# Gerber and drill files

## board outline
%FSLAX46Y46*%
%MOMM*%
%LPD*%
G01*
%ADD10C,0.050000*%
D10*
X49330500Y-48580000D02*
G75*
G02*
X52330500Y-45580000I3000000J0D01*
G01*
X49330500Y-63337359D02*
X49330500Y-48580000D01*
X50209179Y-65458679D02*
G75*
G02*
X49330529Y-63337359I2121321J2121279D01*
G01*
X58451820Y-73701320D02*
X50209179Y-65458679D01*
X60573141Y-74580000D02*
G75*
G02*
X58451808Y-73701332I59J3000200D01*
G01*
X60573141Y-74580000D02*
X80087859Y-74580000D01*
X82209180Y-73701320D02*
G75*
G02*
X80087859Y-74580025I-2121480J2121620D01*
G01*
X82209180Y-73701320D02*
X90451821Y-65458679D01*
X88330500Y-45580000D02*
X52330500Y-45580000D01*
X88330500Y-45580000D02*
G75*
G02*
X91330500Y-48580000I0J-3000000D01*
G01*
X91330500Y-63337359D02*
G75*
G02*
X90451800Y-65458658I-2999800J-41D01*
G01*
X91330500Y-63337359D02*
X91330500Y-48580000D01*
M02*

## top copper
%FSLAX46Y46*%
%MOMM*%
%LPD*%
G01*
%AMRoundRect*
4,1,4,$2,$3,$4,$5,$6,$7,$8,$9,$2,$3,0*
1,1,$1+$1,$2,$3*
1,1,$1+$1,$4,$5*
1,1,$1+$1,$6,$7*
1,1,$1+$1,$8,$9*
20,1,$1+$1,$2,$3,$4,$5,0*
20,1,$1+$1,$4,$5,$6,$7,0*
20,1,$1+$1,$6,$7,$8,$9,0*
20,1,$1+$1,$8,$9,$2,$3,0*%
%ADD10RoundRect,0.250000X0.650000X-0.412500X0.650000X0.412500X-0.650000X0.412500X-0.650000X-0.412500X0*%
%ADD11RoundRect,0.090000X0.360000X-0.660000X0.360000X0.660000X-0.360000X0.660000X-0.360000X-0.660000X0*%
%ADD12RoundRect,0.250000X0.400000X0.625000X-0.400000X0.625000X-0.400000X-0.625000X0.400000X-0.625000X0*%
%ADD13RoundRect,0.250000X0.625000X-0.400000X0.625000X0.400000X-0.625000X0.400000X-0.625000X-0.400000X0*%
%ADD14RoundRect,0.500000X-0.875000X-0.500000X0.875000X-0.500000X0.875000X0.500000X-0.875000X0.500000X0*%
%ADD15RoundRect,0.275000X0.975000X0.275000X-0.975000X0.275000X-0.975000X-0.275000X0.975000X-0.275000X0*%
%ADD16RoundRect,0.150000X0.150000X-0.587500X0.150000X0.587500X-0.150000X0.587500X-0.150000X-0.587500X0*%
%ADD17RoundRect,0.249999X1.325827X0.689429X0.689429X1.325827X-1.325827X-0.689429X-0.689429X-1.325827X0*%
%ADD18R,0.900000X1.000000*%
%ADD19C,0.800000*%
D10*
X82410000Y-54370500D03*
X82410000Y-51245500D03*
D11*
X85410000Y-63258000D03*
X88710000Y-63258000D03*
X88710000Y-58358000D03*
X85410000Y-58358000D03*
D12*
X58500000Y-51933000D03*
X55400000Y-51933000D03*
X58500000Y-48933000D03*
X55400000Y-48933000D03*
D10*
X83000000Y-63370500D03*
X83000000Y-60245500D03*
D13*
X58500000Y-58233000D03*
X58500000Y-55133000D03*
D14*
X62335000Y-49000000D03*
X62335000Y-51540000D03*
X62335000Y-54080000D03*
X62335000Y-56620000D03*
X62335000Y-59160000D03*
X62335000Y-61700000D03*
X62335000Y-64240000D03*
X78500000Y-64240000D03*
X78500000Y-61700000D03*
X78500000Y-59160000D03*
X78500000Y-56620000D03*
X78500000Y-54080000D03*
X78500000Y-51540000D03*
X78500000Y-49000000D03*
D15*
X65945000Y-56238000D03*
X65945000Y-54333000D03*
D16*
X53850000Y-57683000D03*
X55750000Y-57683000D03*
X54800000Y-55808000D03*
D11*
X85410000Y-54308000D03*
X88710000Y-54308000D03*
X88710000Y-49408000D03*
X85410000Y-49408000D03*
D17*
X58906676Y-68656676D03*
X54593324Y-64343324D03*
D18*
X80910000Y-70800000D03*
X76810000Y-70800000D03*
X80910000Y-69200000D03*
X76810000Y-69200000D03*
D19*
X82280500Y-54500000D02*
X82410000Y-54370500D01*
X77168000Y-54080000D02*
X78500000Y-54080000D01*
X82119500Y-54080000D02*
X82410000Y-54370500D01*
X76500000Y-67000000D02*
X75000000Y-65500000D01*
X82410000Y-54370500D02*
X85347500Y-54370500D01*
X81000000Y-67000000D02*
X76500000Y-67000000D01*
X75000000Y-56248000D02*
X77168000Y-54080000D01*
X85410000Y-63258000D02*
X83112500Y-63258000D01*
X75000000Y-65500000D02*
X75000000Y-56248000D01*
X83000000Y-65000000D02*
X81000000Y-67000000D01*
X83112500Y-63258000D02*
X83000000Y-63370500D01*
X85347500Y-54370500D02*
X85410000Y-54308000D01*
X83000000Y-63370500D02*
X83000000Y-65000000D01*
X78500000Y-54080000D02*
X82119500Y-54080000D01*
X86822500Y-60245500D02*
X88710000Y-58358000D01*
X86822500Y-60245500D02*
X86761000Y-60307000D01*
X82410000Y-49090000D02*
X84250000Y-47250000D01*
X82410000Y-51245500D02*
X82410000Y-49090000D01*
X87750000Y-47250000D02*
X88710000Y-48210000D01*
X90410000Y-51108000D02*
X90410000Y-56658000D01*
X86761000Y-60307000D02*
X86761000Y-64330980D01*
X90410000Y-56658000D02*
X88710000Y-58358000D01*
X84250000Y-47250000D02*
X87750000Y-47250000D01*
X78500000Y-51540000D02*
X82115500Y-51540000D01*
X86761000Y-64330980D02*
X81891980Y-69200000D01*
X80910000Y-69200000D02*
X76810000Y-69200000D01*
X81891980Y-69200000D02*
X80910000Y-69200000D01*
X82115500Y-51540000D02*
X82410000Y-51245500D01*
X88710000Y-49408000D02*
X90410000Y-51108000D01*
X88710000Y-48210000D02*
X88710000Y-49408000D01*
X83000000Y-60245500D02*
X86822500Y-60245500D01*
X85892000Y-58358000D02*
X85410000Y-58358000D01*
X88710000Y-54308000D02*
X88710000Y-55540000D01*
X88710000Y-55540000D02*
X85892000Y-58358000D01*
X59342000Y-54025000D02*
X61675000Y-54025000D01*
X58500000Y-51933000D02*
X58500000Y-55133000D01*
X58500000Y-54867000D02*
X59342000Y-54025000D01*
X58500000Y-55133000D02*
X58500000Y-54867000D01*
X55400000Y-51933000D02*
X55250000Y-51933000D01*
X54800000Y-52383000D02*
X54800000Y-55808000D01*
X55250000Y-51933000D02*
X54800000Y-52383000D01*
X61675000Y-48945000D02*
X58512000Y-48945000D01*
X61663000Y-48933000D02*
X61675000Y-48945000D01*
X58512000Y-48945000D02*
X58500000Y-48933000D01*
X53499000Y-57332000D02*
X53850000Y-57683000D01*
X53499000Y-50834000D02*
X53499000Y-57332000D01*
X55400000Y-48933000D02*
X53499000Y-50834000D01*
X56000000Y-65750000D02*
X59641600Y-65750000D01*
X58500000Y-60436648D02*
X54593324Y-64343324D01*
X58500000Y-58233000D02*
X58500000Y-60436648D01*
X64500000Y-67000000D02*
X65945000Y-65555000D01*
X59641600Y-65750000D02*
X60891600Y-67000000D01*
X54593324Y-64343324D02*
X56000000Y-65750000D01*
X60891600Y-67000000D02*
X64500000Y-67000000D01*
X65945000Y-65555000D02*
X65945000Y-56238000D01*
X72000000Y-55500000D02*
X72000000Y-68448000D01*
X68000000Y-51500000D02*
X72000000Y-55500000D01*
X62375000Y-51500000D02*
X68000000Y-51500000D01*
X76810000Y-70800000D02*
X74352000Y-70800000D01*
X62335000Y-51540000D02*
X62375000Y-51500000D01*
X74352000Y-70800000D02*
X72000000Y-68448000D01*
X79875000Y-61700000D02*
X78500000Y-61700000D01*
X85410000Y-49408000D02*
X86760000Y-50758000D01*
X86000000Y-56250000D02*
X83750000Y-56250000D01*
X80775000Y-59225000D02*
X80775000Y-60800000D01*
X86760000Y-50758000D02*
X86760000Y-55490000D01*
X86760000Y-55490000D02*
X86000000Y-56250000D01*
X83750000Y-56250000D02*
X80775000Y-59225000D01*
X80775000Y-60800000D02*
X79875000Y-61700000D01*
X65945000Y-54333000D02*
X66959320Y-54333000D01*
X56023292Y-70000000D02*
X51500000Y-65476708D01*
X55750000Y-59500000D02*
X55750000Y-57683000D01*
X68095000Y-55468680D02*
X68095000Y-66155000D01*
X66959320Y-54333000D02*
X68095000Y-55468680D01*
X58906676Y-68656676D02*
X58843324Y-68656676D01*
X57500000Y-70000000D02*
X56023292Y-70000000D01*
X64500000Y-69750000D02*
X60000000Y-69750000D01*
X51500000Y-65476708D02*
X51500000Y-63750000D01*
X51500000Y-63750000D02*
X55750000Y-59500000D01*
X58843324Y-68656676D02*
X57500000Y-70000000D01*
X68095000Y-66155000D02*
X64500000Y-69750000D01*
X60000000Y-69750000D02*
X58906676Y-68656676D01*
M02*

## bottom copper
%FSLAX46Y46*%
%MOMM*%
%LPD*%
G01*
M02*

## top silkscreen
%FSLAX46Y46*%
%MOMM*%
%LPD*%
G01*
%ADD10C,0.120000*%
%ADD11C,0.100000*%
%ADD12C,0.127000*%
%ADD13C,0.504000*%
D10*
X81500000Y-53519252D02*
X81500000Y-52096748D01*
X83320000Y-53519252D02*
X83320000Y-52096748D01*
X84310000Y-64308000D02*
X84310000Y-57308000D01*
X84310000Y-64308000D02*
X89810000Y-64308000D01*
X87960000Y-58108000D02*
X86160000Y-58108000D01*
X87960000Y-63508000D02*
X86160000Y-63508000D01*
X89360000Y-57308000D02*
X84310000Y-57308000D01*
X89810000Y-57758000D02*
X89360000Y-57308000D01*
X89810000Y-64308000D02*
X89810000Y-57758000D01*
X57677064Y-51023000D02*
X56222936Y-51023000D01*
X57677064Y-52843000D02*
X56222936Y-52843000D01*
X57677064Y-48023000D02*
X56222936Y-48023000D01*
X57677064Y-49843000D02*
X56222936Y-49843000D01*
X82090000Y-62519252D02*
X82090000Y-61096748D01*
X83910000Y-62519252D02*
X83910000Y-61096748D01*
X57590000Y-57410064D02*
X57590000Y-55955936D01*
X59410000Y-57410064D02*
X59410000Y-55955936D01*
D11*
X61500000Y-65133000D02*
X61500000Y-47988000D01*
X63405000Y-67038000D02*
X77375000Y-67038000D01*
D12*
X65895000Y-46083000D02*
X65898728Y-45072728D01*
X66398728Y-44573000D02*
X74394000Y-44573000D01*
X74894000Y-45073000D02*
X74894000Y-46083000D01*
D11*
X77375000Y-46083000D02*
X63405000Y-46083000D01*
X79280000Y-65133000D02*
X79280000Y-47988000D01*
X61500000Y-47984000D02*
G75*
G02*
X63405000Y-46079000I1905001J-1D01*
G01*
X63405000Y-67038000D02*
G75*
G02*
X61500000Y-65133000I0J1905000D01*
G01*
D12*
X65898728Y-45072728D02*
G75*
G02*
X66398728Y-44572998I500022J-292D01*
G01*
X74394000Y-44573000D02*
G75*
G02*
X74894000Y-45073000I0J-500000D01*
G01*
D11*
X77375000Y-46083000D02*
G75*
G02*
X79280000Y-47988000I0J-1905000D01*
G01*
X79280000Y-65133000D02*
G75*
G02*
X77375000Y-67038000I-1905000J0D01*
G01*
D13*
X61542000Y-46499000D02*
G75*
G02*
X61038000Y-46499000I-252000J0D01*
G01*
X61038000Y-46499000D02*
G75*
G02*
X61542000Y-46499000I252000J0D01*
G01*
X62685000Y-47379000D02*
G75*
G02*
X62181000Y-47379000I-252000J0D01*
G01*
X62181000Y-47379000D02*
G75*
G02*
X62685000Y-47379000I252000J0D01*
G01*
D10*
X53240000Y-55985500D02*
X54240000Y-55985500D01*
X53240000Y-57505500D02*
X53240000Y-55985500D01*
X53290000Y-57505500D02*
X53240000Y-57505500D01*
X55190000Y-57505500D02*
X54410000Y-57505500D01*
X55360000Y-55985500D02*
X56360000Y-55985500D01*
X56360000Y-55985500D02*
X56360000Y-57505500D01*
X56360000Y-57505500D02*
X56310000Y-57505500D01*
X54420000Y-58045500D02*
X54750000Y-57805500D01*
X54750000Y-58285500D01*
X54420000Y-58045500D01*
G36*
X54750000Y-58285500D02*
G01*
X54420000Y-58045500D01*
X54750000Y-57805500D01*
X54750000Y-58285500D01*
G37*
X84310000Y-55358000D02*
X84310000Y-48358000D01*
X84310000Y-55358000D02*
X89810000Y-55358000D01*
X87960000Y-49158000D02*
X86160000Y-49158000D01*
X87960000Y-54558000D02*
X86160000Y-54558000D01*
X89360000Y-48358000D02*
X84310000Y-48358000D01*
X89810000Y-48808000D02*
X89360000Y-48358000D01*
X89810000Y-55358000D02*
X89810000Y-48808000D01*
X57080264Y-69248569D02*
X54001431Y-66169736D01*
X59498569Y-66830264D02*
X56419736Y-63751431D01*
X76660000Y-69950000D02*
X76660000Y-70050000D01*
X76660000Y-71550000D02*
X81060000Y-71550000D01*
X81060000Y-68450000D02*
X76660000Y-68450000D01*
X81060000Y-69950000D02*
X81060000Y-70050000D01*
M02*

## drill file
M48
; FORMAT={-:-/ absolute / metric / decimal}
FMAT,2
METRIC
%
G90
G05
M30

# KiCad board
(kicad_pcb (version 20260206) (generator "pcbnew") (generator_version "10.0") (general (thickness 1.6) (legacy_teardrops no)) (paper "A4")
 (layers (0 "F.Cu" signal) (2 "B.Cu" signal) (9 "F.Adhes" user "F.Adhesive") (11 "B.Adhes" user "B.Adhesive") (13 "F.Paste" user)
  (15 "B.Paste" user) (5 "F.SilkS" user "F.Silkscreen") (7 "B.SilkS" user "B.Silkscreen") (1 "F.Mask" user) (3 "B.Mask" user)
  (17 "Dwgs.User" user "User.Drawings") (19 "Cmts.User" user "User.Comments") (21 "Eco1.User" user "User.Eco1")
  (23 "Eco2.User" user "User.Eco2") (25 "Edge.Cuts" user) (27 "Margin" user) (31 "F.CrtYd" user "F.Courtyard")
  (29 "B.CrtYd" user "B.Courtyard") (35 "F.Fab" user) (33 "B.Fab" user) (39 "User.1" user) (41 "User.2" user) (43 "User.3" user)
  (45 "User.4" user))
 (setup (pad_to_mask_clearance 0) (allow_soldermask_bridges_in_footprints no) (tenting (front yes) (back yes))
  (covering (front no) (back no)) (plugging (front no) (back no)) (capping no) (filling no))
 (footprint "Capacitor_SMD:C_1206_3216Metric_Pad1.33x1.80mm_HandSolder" (layer "F.Cu") (at 82.41 52.808 90)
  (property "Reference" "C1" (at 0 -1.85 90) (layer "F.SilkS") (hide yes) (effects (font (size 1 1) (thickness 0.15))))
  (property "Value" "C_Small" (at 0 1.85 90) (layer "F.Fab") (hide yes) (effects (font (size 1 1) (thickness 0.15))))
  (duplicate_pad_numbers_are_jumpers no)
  (fp_line (start -0.711252 -0.91) (end 0.711252 -0.91) (stroke (width 0.12) (type solid)) (layer "F.SilkS"))
  (fp_line (start -0.711252 0.91) (end 0.711252 0.91) (stroke (width 0.12) (type solid)) (layer "F.SilkS"))
  (pad "1" smd roundrect (at -1.5625 0 90) (size 1.325 1.8) (layers "F.Cu" "F.Mask" "F.Paste") (roundrect_rratio 0.188679) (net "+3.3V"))
  (pad "2" smd roundrect (at 1.5625 0 90) (size 1.325 1.8) (layers "F.Cu" "F.Mask" "F.Paste") (roundrect_rratio 0.188679) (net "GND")))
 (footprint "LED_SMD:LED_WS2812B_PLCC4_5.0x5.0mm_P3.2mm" (layer "F.Cu") (at 87.06 60.808 90)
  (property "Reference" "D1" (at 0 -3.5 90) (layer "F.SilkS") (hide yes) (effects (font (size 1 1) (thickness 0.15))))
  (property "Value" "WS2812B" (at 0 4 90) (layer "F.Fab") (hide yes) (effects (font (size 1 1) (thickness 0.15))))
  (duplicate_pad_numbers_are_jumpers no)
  (fp_line (start -3.5 -2.75) (end 3.5 -2.75) (stroke (width 0.12) (type solid)) (layer "F.SilkS"))
  (fp_line (start -3.5 -2.75) (end -3.5 2.75) (stroke (width 0.12) (type default)) (layer "F.SilkS"))
  (fp_line (start 2.7 0.9) (end 2.7 -0.9) (stroke (width 0.12) (type default)) (layer "F.SilkS"))
  (fp_line (start -2.7 0.9) (end -2.7 -0.9) (stroke (width 0.12) (type default)) (layer "F.SilkS"))
  (fp_line (start 3.5 2.3) (end 3.5 -2.75) (stroke (width 0.12) (type default)) (layer "F.SilkS"))
  (fp_line (start 3.05 2.75) (end 3.5 2.3) (stroke (width 0.12) (type default)) (layer "F.SilkS"))
  (fp_line (start -3.5 2.75) (end 3.05 2.75) (stroke (width 0.12) (type solid)) (layer "F.SilkS"))
  (pad "1" smd roundrect (at -2.45 -1.65 90) (size 1.5 0.9) (layers "F.Cu" "F.Mask" "F.Paste") (roundrect_rratio 0.1) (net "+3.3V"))
  (pad "2" smd roundrect (at -2.45 1.65 90) (size 1.5 0.9) (layers "F.Cu" "F.Mask" "F.Paste") (roundrect_rratio 0.1)
   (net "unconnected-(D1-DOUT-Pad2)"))
  (pad "3" smd roundrect (at 2.45 1.65 90) (size 1.5 0.9) (layers "F.Cu" "F.Mask" "F.Paste") (roundrect_rratio 0.1) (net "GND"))
  (pad "4" smd roundrect (at 2.45 -1.65 90) (size 1.5 0.9) (layers "F.Cu" "F.Mask" "F.Paste") (roundrect_rratio 0.1) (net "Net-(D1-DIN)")))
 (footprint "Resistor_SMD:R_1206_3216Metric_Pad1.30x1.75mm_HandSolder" (layer "F.Cu") (at 56.95 51.933 180)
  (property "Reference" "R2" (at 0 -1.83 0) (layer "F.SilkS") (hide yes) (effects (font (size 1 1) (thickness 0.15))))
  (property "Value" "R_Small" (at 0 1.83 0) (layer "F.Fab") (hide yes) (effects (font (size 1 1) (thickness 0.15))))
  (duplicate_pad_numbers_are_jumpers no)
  (fp_line (start -0.727064 0.91) (end 0.727064 0.91) (stroke (width 0.12) (type solid)) (layer "F.SilkS"))
  (fp_line (start -0.727064 -0.91) (end 0.727064 -0.91) (stroke (width 0.12) (type solid)) (layer "F.SilkS"))
  (pad "1" smd roundrect (at -1.55 0 180) (size 1.3 1.75) (layers "F.Cu" "F.Mask" "F.Paste") (roundrect_rratio 0.192308) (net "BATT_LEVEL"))
  (pad "2" smd roundrect (at 1.55 0 180) (size 1.3 1.75) (layers "F.Cu" "F.Mask" "F.Paste") (roundrect_rratio 0.192308) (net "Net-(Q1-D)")))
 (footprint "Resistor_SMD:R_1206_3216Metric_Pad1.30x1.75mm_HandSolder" (layer "F.Cu") (at 56.95 48.933 180)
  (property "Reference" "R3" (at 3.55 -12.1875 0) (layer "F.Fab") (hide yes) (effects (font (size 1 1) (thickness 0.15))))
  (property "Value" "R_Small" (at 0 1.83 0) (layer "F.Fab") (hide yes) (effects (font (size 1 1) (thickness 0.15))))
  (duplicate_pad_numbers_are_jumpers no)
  (fp_line (start -0.727064 0.91) (end 0.727064 0.91) (stroke (width 0.12) (type solid)) (layer "F.SilkS"))
  (fp_line (start -0.727064 -0.91) (end 0.727064 -0.91) (stroke (width 0.12) (type solid)) (layer "F.SilkS"))
  (pad "1" smd roundrect (at -1.55 0 180) (size 1.3 1.75) (layers "F.Cu" "F.Mask" "F.Paste") (roundrect_rratio 0.192308) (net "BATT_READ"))
  (pad "2" smd roundrect (at 1.55 0 180) (size 1.3 1.75) (layers "F.Cu" "F.Mask" "F.Paste") (roundrect_rratio 0.192308) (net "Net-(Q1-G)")))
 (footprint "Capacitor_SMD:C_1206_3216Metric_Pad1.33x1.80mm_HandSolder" (layer "F.Cu") (at 83 61.808 90)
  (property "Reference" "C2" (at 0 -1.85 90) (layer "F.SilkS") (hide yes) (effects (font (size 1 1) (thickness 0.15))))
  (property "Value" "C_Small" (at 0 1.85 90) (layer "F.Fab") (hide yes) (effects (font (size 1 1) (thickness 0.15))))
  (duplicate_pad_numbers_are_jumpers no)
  (fp_line (start -0.711252 -0.91) (end 0.711252 -0.91) (stroke (width 0.12) (type solid)) (layer "F.SilkS"))
  (fp_line (start -0.711252 0.91) (end 0.711252 0.91) (stroke (width 0.12) (type solid)) (layer "F.SilkS"))
  (pad "1" smd roundrect (at -1.5625 0 90) (size 1.325 1.8) (layers "F.Cu" "F.Mask" "F.Paste") (roundrect_rratio 0.188679) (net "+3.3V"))
  (pad "2" smd roundrect (at 1.5625 0 90) (size 1.325 1.8) (layers "F.Cu" "F.Mask" "F.Paste") (roundrect_rratio 0.188679) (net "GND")))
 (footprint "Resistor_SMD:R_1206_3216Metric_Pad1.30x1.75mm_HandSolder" (layer "F.Cu") (at 58.5 56.683 90)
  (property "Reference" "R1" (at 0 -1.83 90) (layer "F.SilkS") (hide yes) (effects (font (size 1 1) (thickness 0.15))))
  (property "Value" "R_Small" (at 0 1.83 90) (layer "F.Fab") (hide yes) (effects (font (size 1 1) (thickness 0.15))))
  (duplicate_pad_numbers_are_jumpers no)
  (fp_line (start -0.727064 -0.91) (end 0.727064 -0.91) (stroke (width 0.12) (type solid)) (layer "F.SilkS"))
  (fp_line (start -0.727064 0.91) (end 0.727064 0.91) (stroke (width 0.12) (type solid)) (layer "F.SilkS"))
  (pad "1" smd roundrect (at -1.55 0 90) (size 1.3 1.75) (layers "F.Cu" "F.Mask" "F.Paste") (roundrect_rratio 0.192308) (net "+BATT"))
  (pad "2" smd roundrect (at 1.55 0 90) (size 1.3 1.75) (layers "F.Cu" "F.Mask" "F.Paste") (roundrect_rratio 0.192308) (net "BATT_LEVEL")))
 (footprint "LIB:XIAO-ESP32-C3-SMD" (layer "F.Cu") (at 61.5 67.12)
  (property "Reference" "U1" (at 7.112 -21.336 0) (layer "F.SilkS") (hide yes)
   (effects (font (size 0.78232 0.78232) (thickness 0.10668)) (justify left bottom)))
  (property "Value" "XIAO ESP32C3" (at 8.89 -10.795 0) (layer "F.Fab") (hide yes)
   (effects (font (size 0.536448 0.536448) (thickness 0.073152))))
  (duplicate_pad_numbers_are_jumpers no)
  (fp_line (start 0 -1.987) (end 0 -19.132) (stroke (width 0.1) (type solid)) (layer "F.SilkS"))
  (fp_line (start 1.905 -0.082) (end 15.875 -0.082) (stroke (width 0.1) (type solid)) (layer "F.SilkS"))
  (fp_line (start 4.395 -21.037) (end 4.398728 -22.047272) (stroke (width 0.127) (type solid)) (layer "F.SilkS"))
  (fp_line (start 4.898728 -22.547) (end 12.894 -22.547) (stroke (width 0.127) (type solid)) (layer "F.SilkS"))
  (fp_line (start 13.394 -22.047) (end 13.394 -21.037) (stroke (width 0.127) (type solid)) (layer "F.SilkS"))
  (fp_line (start 15.875 -21.037) (end 1.905 -21.037) (stroke (width 0.1) (type solid)) (layer "F.SilkS"))
  (fp_line (start 17.78 -1.987) (end 17.78 -19.132) (stroke (width 0.1) (type solid)) (layer "F.SilkS"))
  (fp_arc (start 0 -19.136) (mid 0.557962 -20.483038) (end 1.905 -21.041) (stroke (width 0.1) (type solid)) (layer "F.SilkS"))
  (fp_arc (start 1.905 -0.082) (mid 0.557962 -0.639962) (end 0 -1.987) (stroke (width 0.1) (type solid)) (layer "F.SilkS"))
  (fp_arc (start 4.398728 -22.047272) (mid 4.545272 -22.40064) (end 4.898728 -22.547) (stroke (width 0.127) (type default))
   (layer "F.SilkS"))
  (fp_arc (start 12.894 -22.547) (mid 13.247553 -22.400553) (end 13.394 -22.047) (stroke (width 0.127) (type default)) (layer "F.SilkS"))
  (fp_arc (start 15.875 -21.037) (mid 17.222038 -20.479038) (end 17.78 -19.132) (stroke (width 0.1) (type solid)) (layer "F.SilkS"))
  (fp_arc (start 17.78 -1.987) (mid 17.222038 -0.639962) (end 15.875 -0.082) (stroke (width 0.1) (type solid)) (layer "F.SilkS"))
  (fp_circle (center -0.21 -20.621) (end -0.21 -20.875) (stroke (width 0.5) (type solid)) (fill yes) (layer "F.SilkS"))
  (fp_circle (center 0.933 -19.741) (end 0.933 -19.995) (stroke (width 0.5) (type solid)) (fill yes) (layer "F.SilkS"))
  (pad "1" smd roundrect (at 0.835 -18.12) (size 2.75 2) (layers "F.Cu" "F.Mask" "F.Paste") (roundrect_rratio 0.25) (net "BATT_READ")
   (solder_mask_margin 0.0508) (thermal_bridge_angle 45))
  (pad "2" smd roundrect (at 0.835 -15.58) (size 2.75 2) (layers "F.Cu" "F.Mask" "F.Paste") (roundrect_rratio 0.25) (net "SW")
   (solder_mask_margin 0.0508) (thermal_bridge_angle 45))
  (pad "3" smd roundrect (at 0.835 -13.04) (size 2.75 2) (layers "F.Cu" "F.Mask" "F.Paste") (roundrect_rratio 0.25) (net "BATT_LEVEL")
   (solder_mask_margin 0.0508) (thermal_bridge_angle 45))
  (pad "4" smd roundrect (at 0.835 -10.5) (size 2.75 2) (layers "F.Cu" "F.Mask" "F.Paste") (roundrect_rratio 0.25)
   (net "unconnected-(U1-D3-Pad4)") (solder_mask_margin 0.0508) (thermal_bridge_angle 45))
  (pad "5" smd roundrect (at 0.835 -7.96) (size 2.75 2) (layers "F.Cu" "F.Mask" "F.Paste") (roundrect_rratio 0.25)
   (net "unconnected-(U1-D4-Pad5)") (solder_mask_margin 0.0508) (thermal_bridge_angle 45))
  (pad "6" smd roundrect (at 0.835 -5.42) (size 2.75 2) (layers "F.Cu" "F.Mask" "F.Paste") (roundrect_rratio 0.25)
   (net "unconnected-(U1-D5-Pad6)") (solder_mask_margin 0.0508) (thermal_bridge_angle 45))
  (pad "7" smd roundrect (at 0.835 -2.88) (size 2.75 2) (layers "F.Cu" "F.Mask" "F.Paste") (roundrect_rratio 0.25)
   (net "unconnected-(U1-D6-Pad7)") (solder_mask_margin 0.0508) (thermal_bridge_angle 45))
  (pad "8" smd roundrect (at 17 -2.88) (size 2.75 2) (layers "F.Cu" "F.Mask" "F.Paste") (roundrect_rratio 0.25)
   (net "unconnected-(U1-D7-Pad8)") (solder_mask_margin 0.0508) (thermal_bridge_angle 45))
  (pad "9" smd roundrect (at 17 -5.42) (size 2.75 2) (layers "F.Cu" "F.Mask" "F.Paste") (roundrect_rratio 0.25) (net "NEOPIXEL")
   (solder_mask_margin 0.0508) (thermal_bridge_angle 45))
  (pad "10" smd roundrect (at 17 -7.96) (size 2.75 2) (layers "F.Cu" "F.Mask" "F.Paste") (roundrect_rratio 0.25)
   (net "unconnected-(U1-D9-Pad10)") (solder_mask_margin 0.0508) (thermal_bridge_angle 45))
  (pad "11" smd roundrect (at 17 -10.5) (size 2.75 2) (layers "F.Cu" "F.Mask" "F.Paste") (roundrect_rratio 0.25)
   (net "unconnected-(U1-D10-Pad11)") (solder_mask_margin 0.0508) (thermal_bridge_angle 45))
  (pad "12" smd roundrect (at 17 -13.04) (size 2.75 2) (layers "F.Cu" "F.Mask" "F.Paste") (roundrect_rratio 0.25) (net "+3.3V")
   (solder_mask_margin 0.0508) (thermal_bridge_angle 45))
  (pad "13" smd roundrect (at 17 -15.58) (size 2.75 2) (layers "F.Cu" "F.Mask" "F.Paste") (roundrect_rratio 0.25) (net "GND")
   (solder_mask_margin 0.0508) (thermal_bridge_angle 45))
  (pad "14" smd roundrect (at 17 -18.12) (size 2.75 2) (layers "F.Cu" "F.Mask" "F.Paste") (roundrect_rratio 0.25)
   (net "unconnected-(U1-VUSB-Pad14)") (solder_mask_margin 0.0508) (thermal_bridge_angle 45))
  (pad "15" smd roundrect (at 4.445 -10.882 180) (size 2.5 1.1) (layers "F.Cu" "F.Mask" "F.Paste") (roundrect_rratio 0.25) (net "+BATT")
   (solder_mask_margin 0.0508) (thermal_bridge_angle 45))
  (pad "16" smd roundrect (at 4.445 -12.787 180) (size 2.5 1.1) (layers "F.Cu" "F.Mask" "F.Paste") (roundrect_rratio 0.25) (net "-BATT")
   (solder_mask_margin 0.0508) (thermal_bridge_angle 45)))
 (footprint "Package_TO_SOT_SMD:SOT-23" (layer "F.Cu") (at 54.8 56.7455 90)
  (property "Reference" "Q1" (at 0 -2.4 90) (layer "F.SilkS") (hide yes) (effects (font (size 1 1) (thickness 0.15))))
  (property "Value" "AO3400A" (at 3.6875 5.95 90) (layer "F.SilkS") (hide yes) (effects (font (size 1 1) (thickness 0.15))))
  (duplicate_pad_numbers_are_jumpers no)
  (fp_line (start 0.76 -1.56) (end 0.76 -0.56) (stroke (width 0.12) (type solid)) (layer "F.SilkS"))
  (fp_line (start -0.76 -1.56) (end 0.76 -1.56) (stroke (width 0.12) (type solid)) (layer "F.SilkS"))
  (fp_line (start -0.76 -1.51) (end -0.76 -1.56) (stroke (width 0.12) (type solid)) (layer "F.SilkS"))
  (fp_line (start -0.76 0.39) (end -0.76 -0.39) (stroke (width 0.12) (type solid)) (layer "F.SilkS"))
  (fp_line (start 0.76 0.56) (end 0.76 1.56) (stroke (width 0.12) (type solid)) (layer "F.SilkS"))
  (fp_line (start 0.76 1.56) (end -0.76 1.56) (stroke (width 0.12) (type solid)) (layer "F.SilkS"))
  (fp_line (start -0.76 1.56) (end -0.76 1.51) (stroke (width 0.12) (type solid)) (layer "F.SilkS"))
  (fp_poly (pts (xy -1.3 -0.38) (xy -1.06 -0.05) (xy -1.54 -0.05)) (stroke (width 0.12) (type solid)) (fill yes) (layer "F.SilkS"))
  (pad "1" smd roundrect (at -0.9375 -0.95 90) (size 1.475 0.6) (layers "F.Cu" "F.Mask" "F.Paste") (roundrect_rratio 0.25)
   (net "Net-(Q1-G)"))
  (pad "2" smd roundrect (at -0.9375 0.95 90) (size 1.475 0.6) (layers "F.Cu" "F.Mask" "F.Paste") (roundrect_rratio 0.25) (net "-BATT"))
  (pad "3" smd roundrect (at 0.9375 0 90) (size 1.475 0.6) (layers "F.Cu" "F.Mask" "F.Paste") (roundrect_rratio 0.25) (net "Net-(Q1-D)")))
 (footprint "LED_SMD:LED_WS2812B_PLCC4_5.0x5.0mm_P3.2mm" (layer "F.Cu") (at 87.06 51.858 90)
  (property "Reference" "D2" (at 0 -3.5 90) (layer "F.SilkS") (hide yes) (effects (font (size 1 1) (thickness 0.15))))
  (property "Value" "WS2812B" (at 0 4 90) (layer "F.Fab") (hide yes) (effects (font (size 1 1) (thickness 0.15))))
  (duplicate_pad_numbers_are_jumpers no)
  (fp_line (start -3.5 -2.75) (end 3.5 -2.75) (stroke (width 0.12) (type solid)) (layer "F.SilkS"))
  (fp_line (start -3.5 -2.75) (end -3.5 2.75) (stroke (width 0.12) (type default)) (layer "F.SilkS"))
  (fp_line (start 2.7 0.9) (end 2.7 -0.9) (stroke (width 0.12) (type default)) (layer "F.SilkS"))
  (fp_line (start -2.7 0.9) (end -2.7 -0.9) (stroke (width 0.12) (type default)) (layer "F.SilkS"))
  (fp_line (start 3.5 2.3) (end 3.5 -2.75) (stroke (width 0.12) (type default)) (layer "F.SilkS"))
  (fp_line (start 3.05 2.75) (end 3.5 2.3) (stroke (width 0.12) (type default)) (layer "F.SilkS"))
  (fp_line (start -3.5 2.75) (end 3.05 2.75) (stroke (width 0.12) (type solid)) (layer "F.SilkS"))
  (pad "1" smd roundrect (at -2.45 -1.65 90) (size 1.5 0.9) (layers "F.Cu" "F.Mask" "F.Paste") (roundrect_rratio 0.1) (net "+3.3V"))
  (pad "2" smd roundrect (at -2.45 1.65 90) (size 1.5 0.9) (layers "F.Cu" "F.Mask" "F.Paste") (roundrect_rratio 0.1) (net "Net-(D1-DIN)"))
  (pad "3" smd roundrect (at 2.45 1.65 90) (size 1.5 0.9) (layers "F.Cu" "F.Mask" "F.Paste") (roundrect_rratio 0.1) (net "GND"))
  (pad "4" smd roundrect (at 2.45 -1.65 90) (size 1.5 0.9) (layers "F.Cu" "F.Mask" "F.Paste") (roundrect_rratio 0.1) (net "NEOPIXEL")))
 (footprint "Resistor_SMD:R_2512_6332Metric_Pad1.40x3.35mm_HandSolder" (layer "F.Cu") (at 56.75 66.5 135)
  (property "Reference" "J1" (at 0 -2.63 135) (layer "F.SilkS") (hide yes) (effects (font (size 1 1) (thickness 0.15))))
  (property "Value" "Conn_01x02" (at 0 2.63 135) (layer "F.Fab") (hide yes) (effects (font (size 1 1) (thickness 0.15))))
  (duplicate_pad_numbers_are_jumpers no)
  (fp_line (start -2.177064 -1.71) (end 2.177064 -1.71) (stroke (width 0.12) (type solid)) (layer "F.SilkS"))
  (fp_line (start -2.177064 1.71) (end 2.177064 1.71) (stroke (width 0.12) (type solid)) (layer "F.SilkS"))
  (pad "1" smd roundrect (at -3.05 0 135) (size 1.4 3.35) (layers "F.Cu" "F.Mask" "F.Paste") (roundrect_rratio 0.178571) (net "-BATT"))
  (pad "2" smd roundrect (at 3.05 0 135) (size 1.4 3.35) (layers "F.Cu" "F.Mask" "F.Paste") (roundrect_rratio 0.178571) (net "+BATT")))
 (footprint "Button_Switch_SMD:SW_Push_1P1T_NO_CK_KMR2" (layer "F.Cu") (at 78.86 70 180)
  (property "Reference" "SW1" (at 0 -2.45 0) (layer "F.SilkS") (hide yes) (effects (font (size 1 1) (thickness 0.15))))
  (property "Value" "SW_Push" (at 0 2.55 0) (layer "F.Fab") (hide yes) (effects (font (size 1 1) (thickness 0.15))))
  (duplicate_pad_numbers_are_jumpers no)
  (fp_line (start 2.2 0.05) (end 2.2 -0.05) (stroke (width 0.12) (type solid)) (layer "F.SilkS"))
  (fp_line (start 2.2 -1.55) (end -2.2 -1.55) (stroke (width 0.12) (type solid)) (layer "F.SilkS"))
  (fp_line (start -2.2 1.55) (end 2.2 1.55) (stroke (width 0.12) (type solid)) (layer "F.SilkS"))
  (fp_line (start -2.2 0.05) (end -2.2 -0.05) (stroke (width 0.12) (type solid)) (layer "F.SilkS"))
  (pad "1" smd rect (at -2.05 -0.8 180) (size 0.9 1) (layers "F.Cu" "F.Mask" "F.Paste") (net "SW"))
  (pad "1" smd rect (at 2.05 -0.8 180) (size 0.9 1) (layers "F.Cu" "F.Mask" "F.Paste") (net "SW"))
  (pad "2" smd rect (at -2.05 0.8 180) (size 0.9 1) (layers "F.Cu" "F.Mask" "F.Paste") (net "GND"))
  (pad "2" smd rect (at 2.05 0.8 180) (size 0.9 1) (layers "F.Cu" "F.Mask" "F.Paste") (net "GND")))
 (gr_arc (start 49.3305 48.58) (mid 50.20918 46.45868) (end 52.3305 45.58) (stroke (width 0.05) (type default)) (layer "Edge.Cuts"))
 (gr_line (start 49.3305 63.337359) (end 49.3305 48.58) (stroke (width 0.05) (type default)) (layer "Edge.Cuts"))
 (gr_arc (start 50.209179 65.458679) (mid 49.558861 64.485409) (end 49.3305 63.337359) (stroke (width 0.05) (type default))
  (layer "Edge.Cuts"))
 (gr_line (start 58.45182 73.70132) (end 50.209179 65.458679) (stroke (width 0.05) (type default)) (layer "Edge.Cuts"))
 (gr_arc (start 60.573141 74.58) (mid 59.425096 74.351626) (end 58.45182 73.70132) (stroke (width 0.05) (type default)) (layer "Edge.Cuts"))
 (gr_line (start 60.573141 74.58) (end 80.087859 74.58) (stroke (width 0.05) (type default)) (layer "Edge.Cuts"))
 (gr_arc (start 82.20918 73.70132) (mid 81.235902 74.351616) (end 80.087859 74.58) (stroke (width 0.05) (type default)) (layer "Edge.Cuts"))
 (gr_line (start 82.20918 73.70132) (end 90.451821 65.458679) (stroke (width 0.05) (type default)) (layer "Edge.Cuts"))
 (gr_line (start 88.3305 45.58) (end 52.3305 45.58) (stroke (width 0.05) (type default)) (layer "Edge.Cuts"))
 (gr_arc (start 88.3305 45.58) (mid 90.45182 46.45868) (end 91.3305 48.58) (stroke (width 0.05) (type default)) (layer "Edge.Cuts"))
 (gr_arc (start 91.3305 63.337359) (mid 91.102152 64.485418) (end 90.451821 65.458679) (stroke (width 0.05) (type default))
  (layer "Edge.Cuts"))
 (gr_line (start 91.3305 63.337359) (end 91.3305 48.58) (stroke (width 0.05) (type default)) (layer "Edge.Cuts"))
 (segment (start 82.2805 54.5) (end 82.41 54.3705) (width 0.8) (layer "F.Cu") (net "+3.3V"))
 (segment (start 77.168 54.08) (end 78.5 54.08) (width 0.8) (layer "F.Cu") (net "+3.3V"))
 (segment (start 82.1195 54.08) (end 82.41 54.3705) (width 0.8) (layer "F.Cu") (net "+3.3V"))
 (segment (start 76.5 67) (end 75 65.5) (width 0.8) (layer "F.Cu") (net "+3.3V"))
 (segment (start 82.41 54.3705) (end 85.3475 54.3705) (width 0.8) (layer "F.Cu") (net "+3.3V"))
 (segment (start 81 67) (end 76.5 67) (width 0.8) (layer "F.Cu") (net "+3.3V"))
 (segment (start 75 56.248) (end 77.168 54.08) (width 0.8) (layer "F.Cu") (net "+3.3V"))
 (segment (start 85.41 63.258) (end 83.1125 63.258) (width 0.8) (layer "F.Cu") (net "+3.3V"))
 (segment (start 75 65.5) (end 75 56.248) (width 0.8) (layer "F.Cu") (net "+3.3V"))
 (segment (start 83 65) (end 81 67) (width 0.8) (layer "F.Cu") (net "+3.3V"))
 (segment (start 83.1125 63.258) (end 83 63.3705) (width 0.8) (layer "F.Cu") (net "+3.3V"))
 (segment (start 85.3475 54.3705) (end 85.41 54.308) (width 0.8) (layer "F.Cu") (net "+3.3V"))
 (segment (start 83 63.3705) (end 83 65) (width 0.8) (layer "F.Cu") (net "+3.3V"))
 (segment (start 78.5 54.08) (end 82.1195 54.08) (width 0.8) (layer "F.Cu") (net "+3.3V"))
 (segment (start 86.8225 60.2455) (end 88.71 58.358) (width 0.8) (layer "F.Cu") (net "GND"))
 (segment (start 86.8225 60.2455) (end 86.761 60.307) (width 0.8) (layer "F.Cu") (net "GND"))
 (segment (start 82.41 49.09) (end 84.25 47.25) (width 0.8) (layer "F.Cu") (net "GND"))
 (segment (start 82.41 51.2455) (end 82.41 49.09) (width 0.8) (layer "F.Cu") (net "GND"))
 (segment (start 87.75 47.25) (end 88.71 48.21) (width 0.8) (layer "F.Cu") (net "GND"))
 (segment (start 90.41 51.108) (end 90.41 56.658) (width 0.8) (layer "F.Cu") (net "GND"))
 (segment (start 86.761 60.307) (end 86.761 64.33098) (width 0.8) (layer "F.Cu") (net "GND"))
 (segment (start 90.41 56.658) (end 88.71 58.358) (width 0.8) (layer "F.Cu") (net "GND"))
 (segment (start 84.25 47.25) (end 87.75 47.25) (width 0.8) (layer "F.Cu") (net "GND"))
 (segment (start 78.5 51.54) (end 82.1155 51.54) (width 0.8) (layer "F.Cu") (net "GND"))
 (segment (start 86.761 64.33098) (end 81.89198 69.2) (width 0.8) (layer "F.Cu") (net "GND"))
 (segment (start 80.91 69.2) (end 76.81 69.2) (width 0.8) (layer "F.Cu") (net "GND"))
 (segment (start 81.89198 69.2) (end 80.91 69.2) (width 0.8) (layer "F.Cu") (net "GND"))
 (segment (start 82.1155 51.54) (end 82.41 51.2455) (width 0.8) (layer "F.Cu") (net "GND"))
 (segment (start 88.71 49.408) (end 90.41 51.108) (width 0.8) (layer "F.Cu") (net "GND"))
 (segment (start 88.71 48.21) (end 88.71 49.408) (width 0.8) (layer "F.Cu") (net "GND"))
 (segment (start 83 60.2455) (end 86.8225 60.2455) (width 0.8) (layer "F.Cu") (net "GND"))
 (segment (start 85.892 58.358) (end 85.41 58.358) (width 0.8) (layer "F.Cu") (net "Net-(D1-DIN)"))
 (segment (start 88.71 54.308) (end 88.71 55.54) (width 0.8) (layer "F.Cu") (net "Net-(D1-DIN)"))
 (segment (start 88.71 55.54) (end 85.892 58.358) (width 0.8) (layer "F.Cu") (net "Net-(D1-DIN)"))
 (segment (start 59.342 54.025) (end 61.675 54.025) (width 0.8) (layer "F.Cu") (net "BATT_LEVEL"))
 (segment (start 58.5 51.933) (end 58.5 55.133) (width 0.8) (layer "F.Cu") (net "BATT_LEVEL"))
 (segment (start 58.5 54.867) (end 59.342 54.025) (width 0.8) (layer "F.Cu") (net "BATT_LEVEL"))
 (segment (start 58.5 55.133) (end 58.5 54.867) (width 0.8) (layer "F.Cu") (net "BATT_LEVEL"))
 (segment (start 55.4 51.933) (end 55.25 51.933) (width 0.8) (layer "F.Cu") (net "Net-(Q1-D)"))
 (segment (start 54.8 52.383) (end 54.8 55.808) (width 0.8) (layer "F.Cu") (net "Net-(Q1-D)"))
 (segment (start 55.25 51.933) (end 54.8 52.383) (width 0.8) (layer "F.Cu") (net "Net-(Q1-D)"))
 (segment (start 61.675 48.945) (end 58.512 48.945) (width 0.8) (layer "F.Cu") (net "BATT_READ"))
 (segment (start 61.663 48.933) (end 61.675 48.945) (width 0.8) (layer "F.Cu") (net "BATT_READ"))
 (segment (start 58.512 48.945) (end 58.5 48.933) (width 0.8) (layer "F.Cu") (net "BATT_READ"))
 (segment (start 53.499 57.332) (end 53.85 57.683) (width 0.8) (layer "F.Cu") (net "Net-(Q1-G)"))
 (segment (start 53.499 50.834) (end 53.499 57.332) (width 0.8) (layer "F.Cu") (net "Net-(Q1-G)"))
 (segment (start 55.4 48.933) (end 53.499 50.834) (width 0.8) (layer "F.Cu") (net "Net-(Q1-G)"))
 (segment (start 56 65.75) (end 59.6416 65.75) (width 0.8) (layer "F.Cu") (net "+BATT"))
 (segment (start 58.5 60.436648) (end 54.593324 64.343324) (width 0.8) (layer "F.Cu") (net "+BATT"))
 (segment (start 58.5 58.233) (end 58.5 60.436648) (width 0.8) (layer "F.Cu") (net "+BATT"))
 (segment (start 64.5 67) (end 65.945 65.555) (width 0.8) (layer "F.Cu") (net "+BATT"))
 (segment (start 59.6416 65.75) (end 60.8916 67) (width 0.8) (layer "F.Cu") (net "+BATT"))
 (segment (start 54.593324 64.343324) (end 56 65.75) (width 0.8) (layer "F.Cu") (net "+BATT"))
 (segment (start 60.8916 67) (end 64.5 67) (width 0.8) (layer "F.Cu") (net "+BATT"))
 (segment (start 65.945 65.555) (end 65.945 56.238) (width 0.8) (layer "F.Cu") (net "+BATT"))
 (segment (start 72 55.5) (end 72 68.448) (width 0.8) (layer "F.Cu") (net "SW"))
 (segment (start 68 51.5) (end 72 55.5) (width 0.8) (layer "F.Cu") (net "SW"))
 (segment (start 62.375 51.5) (end 68 51.5) (width 0.8) (layer "F.Cu") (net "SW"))
 (segment (start 76.81 70.8) (end 74.352 70.8) (width 0.8) (layer "F.Cu") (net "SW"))
 (segment (start 62.335 51.54) (end 62.375 51.5) (width 0.8) (layer "F.Cu") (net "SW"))
 (segment (start 74.352 70.8) (end 72 68.448) (width 0.8) (layer "F.Cu") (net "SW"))
 (segment (start 79.875 61.7) (end 78.5 61.7) (width 0.8) (layer "F.Cu") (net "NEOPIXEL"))
 (segment (start 85.41 49.408) (end 86.76 50.758) (width 0.8) (layer "F.Cu") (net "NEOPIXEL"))
 (segment (start 86 56.25) (end 83.75 56.25) (width 0.8) (layer "F.Cu") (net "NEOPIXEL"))
 (segment (start 80.775 59.225) (end 80.775 60.8) (width 0.8) (layer "F.Cu") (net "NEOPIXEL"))
 (segment (start 86.76 50.758) (end 86.76 55.49) (width 0.8) (layer "F.Cu") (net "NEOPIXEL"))
 (segment (start 86.76 55.49) (end 86 56.25) (width 0.8) (layer "F.Cu") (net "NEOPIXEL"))
 (segment (start 83.75 56.25) (end 80.775 59.225) (width 0.8) (layer "F.Cu") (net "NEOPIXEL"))
 (segment (start 80.775 60.8) (end 79.875 61.7) (width 0.8) (layer "F.Cu") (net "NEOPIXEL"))
 (segment (start 65.945 54.333) (end 66.95932 54.333) (width 0.8) (layer "F.Cu") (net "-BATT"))
 (segment (start 56.023292 70) (end 51.5 65.476708) (width 0.8) (layer "F.Cu") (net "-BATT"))
 (segment (start 55.75 59.5) (end 55.75 57.683) (width 0.8) (layer "F.Cu") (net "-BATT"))
 (segment (start 68.095 55.46868) (end 68.095 66.155) (width 0.8) (layer "F.Cu") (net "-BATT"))
 (segment (start 66.95932 54.333) (end 68.095 55.46868) (width 0.8) (layer "F.Cu") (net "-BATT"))
 (segment (start 58.906676 68.656676) (end 58.843324 68.656676) (width 0.8) (layer "F.Cu") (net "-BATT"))
 (segment (start 57.5 70) (end 56.023292 70) (width 0.8) (layer "F.Cu") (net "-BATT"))
 (segment (start 64.5 69.75) (end 60 69.75) (width 0.8) (layer "F.Cu") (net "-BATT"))
 (segment (start 51.5 65.476708) (end 51.5 63.75) (width 0.8) (layer "F.Cu") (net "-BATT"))
 (segment (start 51.5 63.75) (end 55.75 59.5) (width 0.8) (layer "F.Cu") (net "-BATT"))
 (segment (start 58.843324 68.656676) (end 57.5 70) (width 0.8) (layer "F.Cu") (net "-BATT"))
 (segment (start 68.095 66.155) (end 64.5 69.75) (width 0.8) (layer "F.Cu") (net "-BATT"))
 (segment (start 60 69.75) (end 58.906676 68.656676) (width 0.8) (layer "F.Cu") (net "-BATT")))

